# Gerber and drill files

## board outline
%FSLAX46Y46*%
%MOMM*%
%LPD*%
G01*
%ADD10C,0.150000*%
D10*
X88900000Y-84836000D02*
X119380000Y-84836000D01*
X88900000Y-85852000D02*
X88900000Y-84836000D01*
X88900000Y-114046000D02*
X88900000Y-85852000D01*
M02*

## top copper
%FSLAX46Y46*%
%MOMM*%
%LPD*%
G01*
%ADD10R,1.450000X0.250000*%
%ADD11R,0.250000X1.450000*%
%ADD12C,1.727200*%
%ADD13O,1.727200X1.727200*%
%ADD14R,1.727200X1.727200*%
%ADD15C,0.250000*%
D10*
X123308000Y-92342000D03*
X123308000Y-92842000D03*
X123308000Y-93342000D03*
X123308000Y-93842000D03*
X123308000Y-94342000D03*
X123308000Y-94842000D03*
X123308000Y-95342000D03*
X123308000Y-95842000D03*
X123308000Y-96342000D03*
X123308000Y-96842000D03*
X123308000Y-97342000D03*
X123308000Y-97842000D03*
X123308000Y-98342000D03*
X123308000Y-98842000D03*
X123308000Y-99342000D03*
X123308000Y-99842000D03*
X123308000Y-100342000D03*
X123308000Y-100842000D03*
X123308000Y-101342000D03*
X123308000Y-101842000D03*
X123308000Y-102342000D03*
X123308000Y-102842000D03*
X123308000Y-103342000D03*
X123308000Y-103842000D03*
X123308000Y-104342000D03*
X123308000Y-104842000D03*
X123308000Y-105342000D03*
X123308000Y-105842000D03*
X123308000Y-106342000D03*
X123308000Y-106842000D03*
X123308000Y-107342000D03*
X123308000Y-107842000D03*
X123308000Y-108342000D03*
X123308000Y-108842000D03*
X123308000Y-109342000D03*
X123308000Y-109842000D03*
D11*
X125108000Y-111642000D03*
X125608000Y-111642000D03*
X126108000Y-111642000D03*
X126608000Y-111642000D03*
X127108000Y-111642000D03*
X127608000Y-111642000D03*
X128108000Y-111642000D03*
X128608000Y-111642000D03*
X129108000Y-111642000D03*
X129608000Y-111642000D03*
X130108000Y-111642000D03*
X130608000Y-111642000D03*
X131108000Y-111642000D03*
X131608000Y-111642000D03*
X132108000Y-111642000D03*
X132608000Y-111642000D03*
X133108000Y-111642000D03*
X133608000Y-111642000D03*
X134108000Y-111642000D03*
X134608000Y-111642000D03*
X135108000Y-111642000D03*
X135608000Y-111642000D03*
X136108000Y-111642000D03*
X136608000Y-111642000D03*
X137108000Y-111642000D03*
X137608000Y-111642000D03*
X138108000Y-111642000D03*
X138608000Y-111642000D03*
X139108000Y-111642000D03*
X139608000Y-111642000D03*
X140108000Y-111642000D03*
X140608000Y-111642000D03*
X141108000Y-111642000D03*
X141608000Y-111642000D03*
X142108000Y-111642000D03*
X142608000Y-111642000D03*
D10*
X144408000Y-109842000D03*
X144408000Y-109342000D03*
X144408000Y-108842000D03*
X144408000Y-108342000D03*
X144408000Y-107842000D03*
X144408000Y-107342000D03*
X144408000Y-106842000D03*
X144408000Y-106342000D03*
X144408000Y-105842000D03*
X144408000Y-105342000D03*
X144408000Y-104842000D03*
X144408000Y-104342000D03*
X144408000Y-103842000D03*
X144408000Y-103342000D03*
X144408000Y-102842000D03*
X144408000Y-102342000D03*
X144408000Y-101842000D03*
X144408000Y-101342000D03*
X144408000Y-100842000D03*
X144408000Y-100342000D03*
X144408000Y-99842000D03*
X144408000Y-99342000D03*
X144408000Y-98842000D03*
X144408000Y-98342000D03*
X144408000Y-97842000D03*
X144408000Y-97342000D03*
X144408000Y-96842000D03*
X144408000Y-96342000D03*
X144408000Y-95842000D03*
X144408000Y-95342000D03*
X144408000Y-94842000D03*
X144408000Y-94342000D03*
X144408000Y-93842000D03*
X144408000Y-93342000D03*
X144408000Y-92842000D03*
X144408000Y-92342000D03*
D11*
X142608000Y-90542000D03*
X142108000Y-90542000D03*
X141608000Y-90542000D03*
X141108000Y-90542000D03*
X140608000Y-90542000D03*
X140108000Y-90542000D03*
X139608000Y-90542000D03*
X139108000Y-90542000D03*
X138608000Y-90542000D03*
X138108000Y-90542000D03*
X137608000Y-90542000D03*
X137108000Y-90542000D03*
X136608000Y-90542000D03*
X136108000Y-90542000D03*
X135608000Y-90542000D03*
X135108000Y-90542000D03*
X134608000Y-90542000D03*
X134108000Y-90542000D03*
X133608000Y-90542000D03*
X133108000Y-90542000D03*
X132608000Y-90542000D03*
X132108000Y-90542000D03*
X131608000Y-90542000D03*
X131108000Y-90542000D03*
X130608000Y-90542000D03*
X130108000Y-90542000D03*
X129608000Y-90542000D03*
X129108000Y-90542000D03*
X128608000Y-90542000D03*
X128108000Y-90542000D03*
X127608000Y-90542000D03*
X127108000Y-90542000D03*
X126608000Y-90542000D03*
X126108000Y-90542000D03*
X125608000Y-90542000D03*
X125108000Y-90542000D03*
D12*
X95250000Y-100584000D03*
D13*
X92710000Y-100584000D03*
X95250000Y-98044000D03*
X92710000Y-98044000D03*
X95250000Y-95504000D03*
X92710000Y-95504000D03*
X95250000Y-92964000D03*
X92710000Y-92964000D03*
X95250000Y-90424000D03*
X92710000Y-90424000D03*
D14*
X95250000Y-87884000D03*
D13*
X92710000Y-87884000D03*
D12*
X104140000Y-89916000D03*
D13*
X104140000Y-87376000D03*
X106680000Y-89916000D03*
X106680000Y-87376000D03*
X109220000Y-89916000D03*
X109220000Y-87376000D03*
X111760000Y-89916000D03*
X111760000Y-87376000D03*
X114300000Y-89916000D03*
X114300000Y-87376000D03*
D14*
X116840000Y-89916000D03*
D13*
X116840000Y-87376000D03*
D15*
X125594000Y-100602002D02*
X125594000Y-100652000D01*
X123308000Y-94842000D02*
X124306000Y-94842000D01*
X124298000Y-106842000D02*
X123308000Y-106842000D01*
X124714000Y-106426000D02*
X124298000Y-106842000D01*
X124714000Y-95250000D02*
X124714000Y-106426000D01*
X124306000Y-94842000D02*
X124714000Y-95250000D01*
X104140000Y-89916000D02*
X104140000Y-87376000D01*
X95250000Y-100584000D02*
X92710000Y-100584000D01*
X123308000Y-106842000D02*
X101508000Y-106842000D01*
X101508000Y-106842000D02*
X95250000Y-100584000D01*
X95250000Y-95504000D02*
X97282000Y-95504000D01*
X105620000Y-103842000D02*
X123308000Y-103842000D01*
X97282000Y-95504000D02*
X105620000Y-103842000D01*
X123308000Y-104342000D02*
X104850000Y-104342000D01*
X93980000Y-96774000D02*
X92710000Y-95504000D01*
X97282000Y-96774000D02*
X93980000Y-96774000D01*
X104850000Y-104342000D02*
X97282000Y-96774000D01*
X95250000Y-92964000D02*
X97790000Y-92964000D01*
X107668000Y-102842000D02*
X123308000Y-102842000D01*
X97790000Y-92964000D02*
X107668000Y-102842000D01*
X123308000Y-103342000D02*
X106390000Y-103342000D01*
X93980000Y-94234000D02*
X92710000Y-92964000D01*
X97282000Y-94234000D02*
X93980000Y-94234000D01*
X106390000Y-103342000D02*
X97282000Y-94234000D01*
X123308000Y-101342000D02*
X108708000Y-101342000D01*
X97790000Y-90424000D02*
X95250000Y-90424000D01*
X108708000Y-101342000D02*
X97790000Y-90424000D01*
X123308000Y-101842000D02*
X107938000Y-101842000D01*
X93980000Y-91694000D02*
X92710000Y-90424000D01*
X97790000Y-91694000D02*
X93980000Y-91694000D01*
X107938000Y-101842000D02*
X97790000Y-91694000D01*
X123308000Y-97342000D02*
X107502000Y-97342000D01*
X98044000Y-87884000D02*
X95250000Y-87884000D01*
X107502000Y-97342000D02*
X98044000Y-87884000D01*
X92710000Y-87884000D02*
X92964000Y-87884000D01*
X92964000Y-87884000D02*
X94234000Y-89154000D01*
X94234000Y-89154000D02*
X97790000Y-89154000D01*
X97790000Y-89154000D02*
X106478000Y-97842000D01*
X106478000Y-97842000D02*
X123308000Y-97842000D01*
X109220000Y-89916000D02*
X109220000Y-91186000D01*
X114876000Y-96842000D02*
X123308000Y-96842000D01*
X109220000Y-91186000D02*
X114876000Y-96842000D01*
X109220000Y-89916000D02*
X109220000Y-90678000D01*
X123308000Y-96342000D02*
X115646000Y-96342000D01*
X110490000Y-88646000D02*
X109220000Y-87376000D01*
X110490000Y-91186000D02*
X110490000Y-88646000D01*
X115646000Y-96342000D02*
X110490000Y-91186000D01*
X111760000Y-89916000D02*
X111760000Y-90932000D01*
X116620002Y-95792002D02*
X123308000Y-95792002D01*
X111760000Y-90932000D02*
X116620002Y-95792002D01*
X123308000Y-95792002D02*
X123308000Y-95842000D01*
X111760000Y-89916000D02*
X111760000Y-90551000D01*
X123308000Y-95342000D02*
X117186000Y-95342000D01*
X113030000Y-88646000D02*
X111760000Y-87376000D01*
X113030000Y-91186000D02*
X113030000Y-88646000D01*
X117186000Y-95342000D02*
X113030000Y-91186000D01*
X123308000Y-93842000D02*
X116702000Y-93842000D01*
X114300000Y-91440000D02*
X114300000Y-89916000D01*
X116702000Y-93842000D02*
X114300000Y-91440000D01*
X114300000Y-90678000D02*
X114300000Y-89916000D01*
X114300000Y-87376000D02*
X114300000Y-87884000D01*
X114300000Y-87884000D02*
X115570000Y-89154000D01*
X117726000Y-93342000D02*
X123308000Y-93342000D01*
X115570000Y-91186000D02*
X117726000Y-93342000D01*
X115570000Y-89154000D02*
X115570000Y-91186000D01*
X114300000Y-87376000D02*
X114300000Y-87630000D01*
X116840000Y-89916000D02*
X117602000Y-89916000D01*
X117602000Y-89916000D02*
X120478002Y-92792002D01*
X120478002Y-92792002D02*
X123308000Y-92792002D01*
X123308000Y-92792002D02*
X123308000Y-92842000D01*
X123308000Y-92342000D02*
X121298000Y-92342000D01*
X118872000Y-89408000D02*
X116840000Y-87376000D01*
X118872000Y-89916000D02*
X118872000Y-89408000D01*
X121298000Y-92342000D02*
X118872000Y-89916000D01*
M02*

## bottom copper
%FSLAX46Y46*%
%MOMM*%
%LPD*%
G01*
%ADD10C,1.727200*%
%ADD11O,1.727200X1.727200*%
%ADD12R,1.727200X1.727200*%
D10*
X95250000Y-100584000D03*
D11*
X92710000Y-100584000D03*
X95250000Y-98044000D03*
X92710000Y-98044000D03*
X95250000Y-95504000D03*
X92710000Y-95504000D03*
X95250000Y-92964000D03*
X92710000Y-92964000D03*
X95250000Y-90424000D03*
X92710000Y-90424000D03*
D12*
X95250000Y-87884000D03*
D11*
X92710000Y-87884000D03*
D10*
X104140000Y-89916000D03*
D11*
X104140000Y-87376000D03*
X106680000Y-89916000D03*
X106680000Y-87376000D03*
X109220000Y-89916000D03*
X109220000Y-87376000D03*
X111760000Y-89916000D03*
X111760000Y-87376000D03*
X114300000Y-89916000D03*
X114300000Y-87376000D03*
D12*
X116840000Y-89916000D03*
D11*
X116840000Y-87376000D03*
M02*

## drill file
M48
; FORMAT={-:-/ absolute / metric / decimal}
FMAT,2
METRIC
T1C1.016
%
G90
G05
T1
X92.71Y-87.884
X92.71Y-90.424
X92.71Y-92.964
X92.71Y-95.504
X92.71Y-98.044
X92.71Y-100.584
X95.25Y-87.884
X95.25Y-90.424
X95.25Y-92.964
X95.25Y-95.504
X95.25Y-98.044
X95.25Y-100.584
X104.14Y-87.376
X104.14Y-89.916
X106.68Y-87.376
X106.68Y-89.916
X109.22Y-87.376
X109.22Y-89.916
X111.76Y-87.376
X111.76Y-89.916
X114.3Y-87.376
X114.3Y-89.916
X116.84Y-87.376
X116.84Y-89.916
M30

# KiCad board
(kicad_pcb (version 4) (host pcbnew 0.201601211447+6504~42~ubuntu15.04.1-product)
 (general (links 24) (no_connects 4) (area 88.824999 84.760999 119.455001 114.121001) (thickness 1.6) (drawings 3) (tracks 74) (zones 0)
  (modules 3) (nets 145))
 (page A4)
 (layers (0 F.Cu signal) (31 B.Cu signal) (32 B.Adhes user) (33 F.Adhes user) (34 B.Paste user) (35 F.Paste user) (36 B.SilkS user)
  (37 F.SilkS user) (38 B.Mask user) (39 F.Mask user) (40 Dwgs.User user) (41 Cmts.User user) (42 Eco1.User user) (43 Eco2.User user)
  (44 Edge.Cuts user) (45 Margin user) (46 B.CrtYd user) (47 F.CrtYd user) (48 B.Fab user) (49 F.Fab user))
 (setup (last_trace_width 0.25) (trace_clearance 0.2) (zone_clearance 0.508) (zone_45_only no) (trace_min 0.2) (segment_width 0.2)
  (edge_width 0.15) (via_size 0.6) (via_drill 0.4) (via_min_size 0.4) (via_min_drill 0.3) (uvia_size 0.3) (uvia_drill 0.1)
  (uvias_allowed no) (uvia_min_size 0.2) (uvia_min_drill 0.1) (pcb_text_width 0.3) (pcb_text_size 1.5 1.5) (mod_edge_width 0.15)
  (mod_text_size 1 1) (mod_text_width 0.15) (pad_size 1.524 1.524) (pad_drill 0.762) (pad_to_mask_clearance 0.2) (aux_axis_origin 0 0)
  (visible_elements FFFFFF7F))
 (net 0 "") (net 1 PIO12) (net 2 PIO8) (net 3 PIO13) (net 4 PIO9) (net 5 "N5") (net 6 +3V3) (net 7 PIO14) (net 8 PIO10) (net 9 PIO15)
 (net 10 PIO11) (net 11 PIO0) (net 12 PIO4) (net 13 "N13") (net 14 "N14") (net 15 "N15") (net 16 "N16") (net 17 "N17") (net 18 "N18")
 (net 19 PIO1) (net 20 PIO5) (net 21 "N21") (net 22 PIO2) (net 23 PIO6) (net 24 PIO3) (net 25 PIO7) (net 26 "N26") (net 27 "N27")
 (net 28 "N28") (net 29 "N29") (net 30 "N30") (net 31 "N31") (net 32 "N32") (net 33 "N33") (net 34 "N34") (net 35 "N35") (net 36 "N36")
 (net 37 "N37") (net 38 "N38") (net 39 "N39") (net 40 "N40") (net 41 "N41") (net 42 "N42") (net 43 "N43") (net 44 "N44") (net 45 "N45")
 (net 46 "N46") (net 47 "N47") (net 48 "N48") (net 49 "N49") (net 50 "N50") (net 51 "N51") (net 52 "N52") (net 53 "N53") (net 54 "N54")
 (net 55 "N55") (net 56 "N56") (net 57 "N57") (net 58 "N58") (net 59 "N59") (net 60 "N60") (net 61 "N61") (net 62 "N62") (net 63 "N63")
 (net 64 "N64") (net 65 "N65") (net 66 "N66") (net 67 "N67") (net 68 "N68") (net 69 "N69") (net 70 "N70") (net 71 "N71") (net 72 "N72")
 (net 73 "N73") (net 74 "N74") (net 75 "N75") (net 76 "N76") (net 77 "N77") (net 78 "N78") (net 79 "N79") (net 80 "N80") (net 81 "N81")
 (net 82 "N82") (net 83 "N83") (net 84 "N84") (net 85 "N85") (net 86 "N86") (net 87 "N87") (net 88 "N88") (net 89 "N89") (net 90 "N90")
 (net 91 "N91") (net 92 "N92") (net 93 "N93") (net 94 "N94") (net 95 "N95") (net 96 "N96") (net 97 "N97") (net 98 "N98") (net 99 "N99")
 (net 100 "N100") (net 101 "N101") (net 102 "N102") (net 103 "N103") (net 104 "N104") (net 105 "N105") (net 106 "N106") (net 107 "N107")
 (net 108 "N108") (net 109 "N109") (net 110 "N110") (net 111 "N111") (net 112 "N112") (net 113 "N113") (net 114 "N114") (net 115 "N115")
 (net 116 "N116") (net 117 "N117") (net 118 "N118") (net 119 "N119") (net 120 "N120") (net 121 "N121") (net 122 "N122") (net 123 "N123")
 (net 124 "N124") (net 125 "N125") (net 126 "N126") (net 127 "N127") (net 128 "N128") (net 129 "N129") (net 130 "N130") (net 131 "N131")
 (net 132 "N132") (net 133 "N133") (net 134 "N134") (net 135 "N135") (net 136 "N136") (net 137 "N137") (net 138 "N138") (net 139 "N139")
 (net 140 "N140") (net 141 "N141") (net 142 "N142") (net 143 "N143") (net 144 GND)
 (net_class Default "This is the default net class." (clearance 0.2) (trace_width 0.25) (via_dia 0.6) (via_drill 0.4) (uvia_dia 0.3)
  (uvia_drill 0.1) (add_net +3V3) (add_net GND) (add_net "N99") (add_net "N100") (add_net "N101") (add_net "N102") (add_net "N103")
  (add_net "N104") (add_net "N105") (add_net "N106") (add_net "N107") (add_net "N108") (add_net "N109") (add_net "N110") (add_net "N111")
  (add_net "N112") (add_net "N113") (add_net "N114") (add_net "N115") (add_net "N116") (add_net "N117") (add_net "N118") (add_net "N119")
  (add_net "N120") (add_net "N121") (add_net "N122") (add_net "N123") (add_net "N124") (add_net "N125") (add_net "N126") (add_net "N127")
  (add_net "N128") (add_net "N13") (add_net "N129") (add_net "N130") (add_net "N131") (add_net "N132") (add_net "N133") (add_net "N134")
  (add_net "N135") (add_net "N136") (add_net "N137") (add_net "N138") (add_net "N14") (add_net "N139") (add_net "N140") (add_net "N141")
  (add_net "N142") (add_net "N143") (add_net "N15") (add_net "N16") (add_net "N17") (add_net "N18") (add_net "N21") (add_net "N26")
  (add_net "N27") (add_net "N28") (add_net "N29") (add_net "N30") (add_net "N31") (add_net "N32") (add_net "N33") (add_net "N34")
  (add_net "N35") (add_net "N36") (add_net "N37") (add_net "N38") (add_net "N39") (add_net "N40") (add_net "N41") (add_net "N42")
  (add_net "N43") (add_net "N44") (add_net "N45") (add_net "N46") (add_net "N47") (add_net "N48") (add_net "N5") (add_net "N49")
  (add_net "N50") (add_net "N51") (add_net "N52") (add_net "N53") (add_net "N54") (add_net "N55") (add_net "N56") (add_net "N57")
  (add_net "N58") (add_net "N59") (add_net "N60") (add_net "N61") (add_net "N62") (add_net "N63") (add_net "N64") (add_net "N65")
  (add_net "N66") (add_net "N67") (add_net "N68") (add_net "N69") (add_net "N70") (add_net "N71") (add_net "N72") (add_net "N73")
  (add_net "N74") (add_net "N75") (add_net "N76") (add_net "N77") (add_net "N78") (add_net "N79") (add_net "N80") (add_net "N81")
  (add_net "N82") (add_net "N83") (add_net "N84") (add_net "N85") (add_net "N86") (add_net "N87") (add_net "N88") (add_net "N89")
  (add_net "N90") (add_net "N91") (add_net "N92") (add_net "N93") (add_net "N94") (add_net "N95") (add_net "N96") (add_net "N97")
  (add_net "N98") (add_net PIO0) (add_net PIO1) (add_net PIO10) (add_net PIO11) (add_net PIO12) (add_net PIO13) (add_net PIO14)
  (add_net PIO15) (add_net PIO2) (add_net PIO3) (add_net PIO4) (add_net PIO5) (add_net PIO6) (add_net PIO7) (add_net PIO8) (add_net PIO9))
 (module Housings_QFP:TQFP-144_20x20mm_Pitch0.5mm (layer F.Cu) (at 133.858 101.092)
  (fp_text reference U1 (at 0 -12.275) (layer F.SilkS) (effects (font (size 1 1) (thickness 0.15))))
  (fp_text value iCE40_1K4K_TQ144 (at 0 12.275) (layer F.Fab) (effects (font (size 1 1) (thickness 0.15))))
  (pad 1 smd rect (at -10.55 -8.75) (size 1.45 0.25) (layers F.Cu F.Paste F.Mask) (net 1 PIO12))
  (pad 2 smd rect (at -10.55 -8.25) (size 1.45 0.25) (layers F.Cu F.Paste F.Mask) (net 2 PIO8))
  (pad 3 smd rect (at -10.55 -7.75) (size 1.45 0.25) (layers F.Cu F.Paste F.Mask) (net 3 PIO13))
  (pad 4 smd rect (at -10.55 -7.25) (size 1.45 0.25) (layers F.Cu F.Paste F.Mask) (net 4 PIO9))
  (pad 5 smd rect (at -10.55 -6.75) (size 1.45 0.25) (layers F.Cu F.Paste F.Mask) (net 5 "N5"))
  (pad 6 smd rect (at -10.55 -6.25) (size 1.45 0.25) (layers F.Cu F.Paste F.Mask) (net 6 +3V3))
  (pad 7 smd rect (at -10.55 -5.75) (size 1.45 0.25) (layers F.Cu F.Paste F.Mask) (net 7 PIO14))
  (pad 8 smd rect (at -10.55 -5.25) (size 1.45 0.25) (layers F.Cu F.Paste F.Mask) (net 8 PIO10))
  (pad 9 smd rect (at -10.55 -4.75) (size 1.45 0.25) (layers F.Cu F.Paste F.Mask) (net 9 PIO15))
  (pad 10 smd rect (at -10.55 -4.25) (size 1.45 0.25) (layers F.Cu F.Paste F.Mask) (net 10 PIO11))
  (pad 11 smd rect (at -10.55 -3.75) (size 1.45 0.25) (layers F.Cu F.Paste F.Mask) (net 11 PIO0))
  (pad 12 smd rect (at -10.55 -3.25) (size 1.45 0.25) (layers F.Cu F.Paste F.Mask) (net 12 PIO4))
  (pad 13 smd rect (at -10.55 -2.75) (size 1.45 0.25) (layers F.Cu F.Paste F.Mask) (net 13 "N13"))
  (pad 14 smd rect (at -10.55 -2.25) (size 1.45 0.25) (layers F.Cu F.Paste F.Mask) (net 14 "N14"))
  (pad 15 smd rect (at -10.55 -1.75) (size 1.45 0.25) (layers F.Cu F.Paste F.Mask) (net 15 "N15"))
  (pad 16 smd rect (at -10.55 -1.25) (size 1.45 0.25) (layers F.Cu F.Paste F.Mask) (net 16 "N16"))
  (pad 17 smd rect (at -10.55 -0.75) (size 1.45 0.25) (layers F.Cu F.Paste F.Mask) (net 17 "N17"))
  (pad 18 smd rect (at -10.55 -0.25) (size 1.45 0.25) (layers F.Cu F.Paste F.Mask) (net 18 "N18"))
  (pad 19 smd rect (at -10.55 0.25) (size 1.45 0.25) (layers F.Cu F.Paste F.Mask) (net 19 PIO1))
  (pad 20 smd rect (at -10.55 0.75) (size 1.45 0.25) (layers F.Cu F.Paste F.Mask) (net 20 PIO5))
  (pad 21 smd rect (at -10.55 1.25) (size 1.45 0.25) (layers F.Cu F.Paste F.Mask) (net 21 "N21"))
  (pad 22 smd rect (at -10.55 1.75) (size 1.45 0.25) (layers F.Cu F.Paste F.Mask) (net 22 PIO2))
  (pad 23 smd rect (at -10.55 2.25) (size 1.45 0.25) (layers F.Cu F.Paste F.Mask) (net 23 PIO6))
  (pad 24 smd rect (at -10.55 2.75) (size 1.45 0.25) (layers F.Cu F.Paste F.Mask) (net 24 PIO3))
  (pad 25 smd rect (at -10.55 3.25) (size 1.45 0.25) (layers F.Cu F.Paste F.Mask) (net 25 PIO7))
  (pad 26 smd rect (at -10.55 3.75) (size 1.45 0.25) (layers F.Cu F.Paste F.Mask) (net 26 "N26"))
  (pad 27 smd rect (at -10.55 4.25) (size 1.45 0.25) (layers F.Cu F.Paste F.Mask) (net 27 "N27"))
  (pad 28 smd rect (at -10.55 4.75) (size 1.45 0.25) (layers F.Cu F.Paste F.Mask) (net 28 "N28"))
  (pad 29 smd rect (at -10.55 5.25) (size 1.45 0.25) (layers F.Cu F.Paste F.Mask) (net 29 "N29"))
  (pad 30 smd rect (at -10.55 5.75) (size 1.45 0.25) (layers F.Cu F.Paste F.Mask) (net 6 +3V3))
  (pad 31 smd rect (at -10.55 6.25) (size 1.45 0.25) (layers F.Cu F.Paste F.Mask) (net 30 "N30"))
  (pad 32 smd rect (at -10.55 6.75) (size 1.45 0.25) (layers F.Cu F.Paste F.Mask) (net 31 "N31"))
  (pad 33 smd rect (at -10.55 7.25) (size 1.45 0.25) (layers F.Cu F.Paste F.Mask) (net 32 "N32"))
  (pad 34 smd rect (at -10.55 7.75) (size 1.45 0.25) (layers F.Cu F.Paste F.Mask) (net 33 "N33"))
  (pad 35 smd rect (at -10.55 8.25) (size 1.45 0.25) (layers F.Cu F.Paste F.Mask) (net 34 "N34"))
  (pad 36 smd rect (at -10.55 8.75) (size 1.45 0.25) (layers F.Cu F.Paste F.Mask) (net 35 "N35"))
  (pad 37 smd rect (at -8.75 10.55 90) (size 1.45 0.25) (layers F.Cu F.Paste F.Mask) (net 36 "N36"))
  (pad 38 smd rect (at -8.25 10.55 90) (size 1.45 0.25) (layers F.Cu F.Paste F.Mask) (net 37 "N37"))
  (pad 39 smd rect (at -7.75 10.55 90) (size 1.45 0.25) (layers F.Cu F.Paste F.Mask) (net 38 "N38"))
  (pad 40 smd rect (at -7.25 10.55 90) (size 1.45 0.25) (layers F.Cu F.Paste F.Mask) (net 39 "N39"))
  (pad 41 smd rect (at -6.75 10.55 90) (size 1.45 0.25) (layers F.Cu F.Paste F.Mask) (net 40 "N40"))
  (pad 42 smd rect (at -6.25 10.55 90) (size 1.45 0.25) (layers F.Cu F.Paste F.Mask) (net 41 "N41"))
  (pad 43 smd rect (at -5.75 10.55 90) (size 1.45 0.25) (layers F.Cu F.Paste F.Mask) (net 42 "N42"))
  (pad 44 smd rect (at -5.25 10.55 90) (size 1.45 0.25) (layers F.Cu F.Paste F.Mask) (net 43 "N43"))
  (pad 45 smd rect (at -4.75 10.55 90) (size 1.45 0.25) (layers F.Cu F.Paste F.Mask) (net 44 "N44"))
  (pad 46 smd rect (at -4.25 10.55 90) (size 1.45 0.25) (layers F.Cu F.Paste F.Mask) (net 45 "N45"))
  (pad 47 smd rect (at -3.75 10.55 90) (size 1.45 0.25) (layers F.Cu F.Paste F.Mask) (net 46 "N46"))
  (pad 48 smd rect (at -3.25 10.55 90) (size 1.45 0.25) (layers F.Cu F.Paste F.Mask) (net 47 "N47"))
  (pad 49 smd rect (at -2.75 10.55 90) (size 1.45 0.25) (layers F.Cu F.Paste F.Mask) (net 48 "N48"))
  (pad 50 smd rect (at -2.25 10.55 90) (size 1.45 0.25) (layers F.Cu F.Paste F.Mask) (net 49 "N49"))
  (pad 51 smd rect (at -1.75 10.55 90) (size 1.45 0.25) (layers F.Cu F.Paste F.Mask) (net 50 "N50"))
  (pad 52 smd rect (at -1.25 10.55 90) (size 1.45 0.25) (layers F.Cu F.Paste F.Mask) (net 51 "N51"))
  (pad 53 smd rect (at -0.75 10.55 90) (size 1.45 0.25) (layers F.Cu F.Paste F.Mask) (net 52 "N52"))
  (pad 54 smd rect (at -0.25 10.55 90) (size 1.45 0.25) (layers F.Cu F.Paste F.Mask) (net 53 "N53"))
  (pad 55 smd rect (at 0.25 10.55 90) (size 1.45 0.25) (layers F.Cu F.Paste F.Mask) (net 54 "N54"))
  (pad 56 smd rect (at 0.75 10.55 90) (size 1.45 0.25) (layers F.Cu F.Paste F.Mask) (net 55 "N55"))
  (pad 57 smd rect (at 1.25 10.55 90) (size 1.45 0.25) (layers F.Cu F.Paste F.Mask) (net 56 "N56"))
  (pad 58 smd rect (at 1.75 10.55 90) (size 1.45 0.25) (layers F.Cu F.Paste F.Mask) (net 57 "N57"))
  (pad 59 smd rect (at 2.25 10.55 90) (size 1.45 0.25) (layers F.Cu F.Paste F.Mask) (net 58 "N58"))
  (pad 60 smd rect (at 2.75 10.55 90) (size 1.45 0.25) (layers F.Cu F.Paste F.Mask) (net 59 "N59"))
  (pad 61 smd rect (at 3.25 10.55 90) (size 1.45 0.25) (layers F.Cu F.Paste F.Mask) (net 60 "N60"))
  (pad 62 smd rect (at 3.75 10.55 90) (size 1.45 0.25) (layers F.Cu F.Paste F.Mask) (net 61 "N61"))
  (pad 63 smd rect (at 4.25 10.55 90) (size 1.45 0.25) (layers F.Cu F.Paste F.Mask) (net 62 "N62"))
  (pad 64 smd rect (at 4.75 10.55 90) (size 1.45 0.25) (layers F.Cu F.Paste F.Mask) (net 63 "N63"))
  (pad 65 smd rect (at 5.25 10.55 90) (size 1.45 0.25) (layers F.Cu F.Paste F.Mask) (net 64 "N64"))
  (pad 66 smd rect (at 5.75 10.55 90) (size 1.45 0.25) (layers F.Cu F.Paste F.Mask) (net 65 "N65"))
  (pad 67 smd rect (at 6.25 10.55 90) (size 1.45 0.25) (layers F.Cu F.Paste F.Mask) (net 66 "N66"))
  (pad 68 smd rect (at 6.75 10.55 90) (size 1.45 0.25) (layers F.Cu F.Paste F.Mask) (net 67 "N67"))
  (pad 69 smd rect (at 7.25 10.55 90) (size 1.45 0.25) (layers F.Cu F.Paste F.Mask) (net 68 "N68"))
  (pad 70 smd rect (at 7.75 10.55 90) (size 1.45 0.25) (layers F.Cu F.Paste F.Mask) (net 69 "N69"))
  (pad 71 smd rect (at 8.25 10.55 90) (size 1.45 0.25) (layers F.Cu F.Paste F.Mask) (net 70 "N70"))
  (pad 72 smd rect (at 8.75 10.55 90) (size 1.45 0.25) (layers F.Cu F.Paste F.Mask) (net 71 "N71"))
  (pad 73 smd rect (at 10.55 8.75) (size 1.45 0.25) (layers F.Cu F.Paste F.Mask) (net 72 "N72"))
  (pad 74 smd rect (at 10.55 8.25) (size 1.45 0.25) (layers F.Cu F.Paste F.Mask) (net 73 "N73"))
  (pad 75 smd rect (at 10.55 7.75) (size 1.45 0.25) (layers F.Cu F.Paste F.Mask) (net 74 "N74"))
  (pad 76 smd rect (at 10.55 7.25) (size 1.45 0.25) (layers F.Cu F.Paste F.Mask) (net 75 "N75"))
  (pad 77 smd rect (at 10.55 6.75) (size 1.45 0.25) (layers F.Cu F.Paste F.Mask) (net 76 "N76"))
  (pad 78 smd rect (at 10.55 6.25) (size 1.45 0.25) (layers F.Cu F.Paste F.Mask) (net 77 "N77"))
  (pad 79 smd rect (at 10.55 5.75) (size 1.45 0.25) (layers F.Cu F.Paste F.Mask) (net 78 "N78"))
  (pad 80 smd rect (at 10.55 5.25) (size 1.45 0.25) (layers F.Cu F.Paste F.Mask) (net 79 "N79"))
  (pad 81 smd rect (at 10.55 4.75) (size 1.45 0.25) (layers F.Cu F.Paste F.Mask) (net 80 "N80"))
  (pad 82 smd rect (at 10.55 4.25) (size 1.45 0.25) (layers F.Cu F.Paste F.Mask) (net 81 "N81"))
  (pad 83 smd rect (at 10.55 3.75) (size 1.45 0.25) (layers F.Cu F.Paste F.Mask) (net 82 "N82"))
  (pad 84 smd rect (at 10.55 3.25) (size 1.45 0.25) (layers F.Cu F.Paste F.Mask) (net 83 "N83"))
  (pad 85 smd rect (at 10.55 2.75) (size 1.45 0.25) (layers F.Cu F.Paste F.Mask) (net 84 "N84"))
  (pad 86 smd rect (at 10.55 2.25) (size 1.45 0.25) (layers F.Cu F.Paste F.Mask) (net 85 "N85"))
  (pad 87 smd rect (at 10.55 1.75) (size 1.45 0.25) (layers F.Cu F.Paste F.Mask) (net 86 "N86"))
  (pad 88 smd rect (at 10.55 1.25) (size 1.45 0.25) (layers F.Cu F.Paste F.Mask) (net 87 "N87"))
  (pad 89 smd rect (at 10.55 0.75) (size 1.45 0.25) (layers F.Cu F.Paste F.Mask) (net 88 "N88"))
  (pad 90 smd rect (at 10.55 0.25) (size 1.45 0.25) (layers F.Cu F.Paste F.Mask) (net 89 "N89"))
  (pad 91 smd rect (at 10.55 -0.25) (size 1.45 0.25) (layers F.Cu F.Paste F.Mask) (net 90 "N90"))
  (pad 92 smd rect (at 10.55 -0.75) (size 1.45 0.25) (layers F.Cu F.Paste F.Mask) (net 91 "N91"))
  (pad 93 smd rect (at 10.55 -1.25) (size 1.45 0.25) (layers F.Cu F.Paste F.Mask) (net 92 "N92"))
  (pad 94 smd rect (at 10.55 -1.75) (size 1.45 0.25) (layers F.Cu F.Paste F.Mask) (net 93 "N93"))
  (pad 95 smd rect (at 10.55 -2.25) (size 1.45 0.25) (layers F.Cu F.Paste F.Mask) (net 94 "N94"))
  (pad 96 smd rect (at 10.55 -2.75) (size 1.45 0.25) (layers F.Cu F.Paste F.Mask) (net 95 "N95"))
  (pad 97 smd rect (at 10.55 -3.25) (size 1.45 0.25) (layers F.Cu F.Paste F.Mask) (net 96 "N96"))
  (pad 98 smd rect (at 10.55 -3.75) (size 1.45 0.25) (layers F.Cu F.Paste F.Mask) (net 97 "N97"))
  (pad 99 smd rect (at 10.55 -4.25) (size 1.45 0.25) (layers F.Cu F.Paste F.Mask) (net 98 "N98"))
  (pad 100 smd rect (at 10.55 -4.75) (size 1.45 0.25) (layers F.Cu F.Paste F.Mask) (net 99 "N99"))
  (pad 101 smd rect (at 10.55 -5.25) (size 1.45 0.25) (layers F.Cu F.Paste F.Mask) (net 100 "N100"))
  (pad 102 smd rect (at 10.55 -5.75) (size 1.45 0.25) (layers F.Cu F.Paste F.Mask) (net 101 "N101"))
  (pad 103 smd rect (at 10.55 -6.25) (size 1.45 0.25) (layers F.Cu F.Paste F.Mask) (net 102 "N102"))
  (pad 104 smd rect (at 10.55 -6.75) (size 1.45 0.25) (layers F.Cu F.Paste F.Mask) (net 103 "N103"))
  (pad 105 smd rect (at 10.55 -7.25) (size 1.45 0.25) (layers F.Cu F.Paste F.Mask) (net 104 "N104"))
  (pad 106 smd rect (at 10.55 -7.75) (size 1.45 0.25) (layers F.Cu F.Paste F.Mask) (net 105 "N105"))
  (pad 107 smd rect (at 10.55 -8.25) (size 1.45 0.25) (layers F.Cu F.Paste F.Mask) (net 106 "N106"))
  (pad 108 smd rect (at 10.55 -8.75) (size 1.45 0.25) (layers F.Cu F.Paste F.Mask) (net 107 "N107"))
  (pad 109 smd rect (at 8.75 -10.55 90) (size 1.45 0.25) (layers F.Cu F.Paste F.Mask) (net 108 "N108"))
  (pad 110 smd rect (at 8.25 -10.55 90) (size 1.45 0.25) (layers F.Cu F.Paste F.Mask) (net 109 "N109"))
  (pad 111 smd rect (at 7.75 -10.55 90) (size 1.45 0.25) (layers F.Cu F.Paste F.Mask) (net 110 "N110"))
  (pad 112 smd rect (at 7.25 -10.55 90) (size 1.45 0.25) (layers F.Cu F.Paste F.Mask) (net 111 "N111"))
  (pad 113 smd rect (at 6.75 -10.55 90) (size 1.45 0.25) (layers F.Cu F.Paste F.Mask) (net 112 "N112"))
  (pad 114 smd rect (at 6.25 -10.55 90) (size 1.45 0.25) (layers F.Cu F.Paste F.Mask) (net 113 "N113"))
  (pad 115 smd rect (at 5.75 -10.55 90) (size 1.45 0.25) (layers F.Cu F.Paste F.Mask) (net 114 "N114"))
  (pad 116 smd rect (at 5.25 -10.55 90) (size 1.45 0.25) (layers F.Cu F.Paste F.Mask) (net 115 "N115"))
  (pad 117 smd rect (at 4.75 -10.55 90) (size 1.45 0.25) (layers F.Cu F.Paste F.Mask) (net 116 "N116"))
  (pad 118 smd rect (at 4.25 -10.55 90) (size 1.45 0.25) (layers F.Cu F.Paste F.Mask) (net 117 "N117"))
  (pad 119 smd rect (at 3.75 -10.55 90) (size 1.45 0.25) (layers F.Cu F.Paste F.Mask) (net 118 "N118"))
  (pad 120 smd rect (at 3.25 -10.55 90) (size 1.45 0.25) (layers F.Cu F.Paste F.Mask) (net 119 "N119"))
  (pad 121 smd rect (at 2.75 -10.55 90) (size 1.45 0.25) (layers F.Cu F.Paste F.Mask) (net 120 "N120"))
  (pad 122 smd rect (at 2.25 -10.55 90) (size 1.45 0.25) (layers F.Cu F.Paste F.Mask) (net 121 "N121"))
  (pad 123 smd rect (at 1.75 -10.55 90) (size 1.45 0.25) (layers F.Cu F.Paste F.Mask) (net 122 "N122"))
  (pad 124 smd rect (at 1.25 -10.55 90) (size 1.45 0.25) (layers F.Cu F.Paste F.Mask) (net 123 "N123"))
  (pad 125 smd rect (at 0.75 -10.55 90) (size 1.45 0.25) (layers F.Cu F.Paste F.Mask) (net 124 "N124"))
  (pad 126 smd rect (at 0.25 -10.55 90) (size 1.45 0.25) (layers F.Cu F.Paste F.Mask) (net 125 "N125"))
  (pad 127 smd rect (at -0.25 -10.55 90) (size 1.45 0.25) (layers F.Cu F.Paste F.Mask) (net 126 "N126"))
  (pad 128 smd rect (at -0.75 -10.55 90) (size 1.45 0.25) (layers F.Cu F.Paste F.Mask) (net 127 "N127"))
  (pad 129 smd rect (at -1.25 -10.55 90) (size 1.45 0.25) (layers F.Cu F.Paste F.Mask) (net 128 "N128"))
  (pad 130 smd rect (at -1.75 -10.55 90) (size 1.45 0.25) (layers F.Cu F.Paste F.Mask) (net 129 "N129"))
  (pad 131 smd rect (at -2.25 -10.55 90) (size 1.45 0.25) (layers F.Cu F.Paste F.Mask) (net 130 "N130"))
  (pad 132 smd rect (at -2.75 -10.55 90) (size 1.45 0.25) (layers F.Cu F.Paste F.Mask) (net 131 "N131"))
  (pad 133 smd rect (at -3.25 -10.55 90) (size 1.45 0.25) (layers F.Cu F.Paste F.Mask) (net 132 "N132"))
  (pad 134 smd rect (at -3.75 -10.55 90) (size 1.45 0.25) (layers F.Cu F.Paste F.Mask) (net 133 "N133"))
  (pad 135 smd rect (at -4.25 -10.55 90) (size 1.45 0.25) (layers F.Cu F.Paste F.Mask) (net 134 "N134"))
  (pad 136 smd rect (at -4.75 -10.55 90) (size 1.45 0.25) (layers F.Cu F.Paste F.Mask) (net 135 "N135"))
  (pad 137 smd rect (at -5.25 -10.55 90) (size 1.45 0.25) (layers F.Cu F.Paste F.Mask) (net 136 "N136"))
  (pad 138 smd rect (at -5.75 -10.55 90) (size 1.45 0.25) (layers F.Cu F.Paste F.Mask) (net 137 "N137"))
  (pad 139 smd rect (at -6.25 -10.55 90) (size 1.45 0.25) (layers F.Cu F.Paste F.Mask) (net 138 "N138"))
  (pad 140 smd rect (at -6.75 -10.55 90) (size 1.45 0.25) (layers F.Cu F.Paste F.Mask) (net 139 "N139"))
  (pad 141 smd rect (at -7.25 -10.55 90) (size 1.45 0.25) (layers F.Cu F.Paste F.Mask) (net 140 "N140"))
  (pad 142 smd rect (at -7.75 -10.55 90) (size 1.45 0.25) (layers F.Cu F.Paste F.Mask) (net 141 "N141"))
  (pad 143 smd rect (at -8.25 -10.55 90) (size 1.45 0.25) (layers F.Cu F.Paste F.Mask) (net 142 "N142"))
  (pad 144 smd rect (at -8.75 -10.55 90) (size 1.45 0.25) (layers F.Cu F.Paste F.Mask) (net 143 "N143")))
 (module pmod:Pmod (layer F.Cu) (at 88.9 86.614)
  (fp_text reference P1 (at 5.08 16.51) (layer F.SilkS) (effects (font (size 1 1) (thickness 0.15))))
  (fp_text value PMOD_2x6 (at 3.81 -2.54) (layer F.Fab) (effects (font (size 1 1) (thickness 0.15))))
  (pad 6 thru_hole circle (at 6.35 13.97 180) (size 1.7272 1.7272) (drill 1.016) (layers *.Cu *.Mask F.SilkS) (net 6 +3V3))
  (pad 12 thru_hole oval (at 3.81 13.97 180) (size 1.7272 1.7272) (drill 1.016) (layers *.Cu *.Mask F.SilkS) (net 6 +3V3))
  (pad 5 thru_hole oval (at 6.35 11.43 180) (size 1.7272 1.7272) (drill 1.016) (layers *.Cu *.Mask F.SilkS) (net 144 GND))
  (pad 11 thru_hole oval (at 3.81 11.43 180) (size 1.7272 1.7272) (drill 1.016) (layers *.Cu *.Mask F.SilkS) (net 144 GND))
  (pad 4 thru_hole oval (at 6.35 8.89 180) (size 1.7272 1.7272) (drill 1.016) (layers *.Cu *.Mask F.SilkS) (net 24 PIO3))
  (pad 10 thru_hole oval (at 3.81 8.89 180) (size 1.7272 1.7272) (drill 1.016) (layers *.Cu *.Mask F.SilkS) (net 25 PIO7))
  (pad 3 thru_hole oval (at 6.35 6.35 180) (size 1.7272 1.7272) (drill 1.016) (layers *.Cu *.Mask F.SilkS) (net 22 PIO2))
  (pad 9 thru_hole oval (at 3.81 6.35 180) (size 1.7272 1.7272) (drill 1.016) (layers *.Cu *.Mask F.SilkS) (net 23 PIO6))
  (pad 2 thru_hole oval (at 6.35 3.81 180) (size 1.7272 1.7272) (drill 1.016) (layers *.Cu *.Mask F.SilkS) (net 19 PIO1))
  (pad 8 thru_hole oval (at 3.81 3.81 180) (size 1.7272 1.7272) (drill 1.016) (layers *.Cu *.Mask F.SilkS) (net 20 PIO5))
  (pad 1 thru_hole rect (at 6.35 1.27 180) (size 1.7272 1.7272) (drill 1.016) (layers *.Cu *.Mask F.SilkS) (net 11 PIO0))
  (pad 7 thru_hole oval (at 3.81 1.27 180) (size 1.7272 1.7272) (drill 1.016) (layers *.Cu *.Mask F.SilkS) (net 12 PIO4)))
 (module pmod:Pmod (layer F.Cu) (at 118.11 83.566 270)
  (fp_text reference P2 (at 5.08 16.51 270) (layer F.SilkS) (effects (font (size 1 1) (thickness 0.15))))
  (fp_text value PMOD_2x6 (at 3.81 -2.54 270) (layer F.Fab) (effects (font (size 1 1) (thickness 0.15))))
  (pad 6 thru_hole circle (at 6.35 13.97 90) (size 1.7272 1.7272) (drill 1.016) (layers *.Cu *.Mask F.SilkS) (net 6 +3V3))
  (pad 12 thru_hole oval (at 3.81 13.97 90) (size 1.7272 1.7272) (drill 1.016) (layers *.Cu *.Mask F.SilkS) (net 6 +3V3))
  (pad 5 thru_hole oval (at 6.35 11.43 90) (size 1.7272 1.7272) (drill 1.016) (layers *.Cu *.Mask F.SilkS) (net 144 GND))
  (pad 11 thru_hole oval (at 3.81 11.43 90) (size 1.7272 1.7272) (drill 1.016) (layers *.Cu *.Mask F.SilkS) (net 144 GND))
  (pad 4 thru_hole oval (at 6.35 8.89 90) (size 1.7272 1.7272) (drill 1.016) (layers *.Cu *.Mask F.SilkS) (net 10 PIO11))
  (pad 10 thru_hole oval (at 3.81 8.89 90) (size 1.7272 1.7272) (drill 1.016) (layers *.Cu *.Mask F.SilkS) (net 9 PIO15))
  (pad 3 thru_hole oval (at 6.35 6.35 90) (size 1.7272 1.7272) (drill 1.016) (layers *.Cu *.Mask F.SilkS) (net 8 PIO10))
  (pad 9 thru_hole oval (at 3.81 6.35 90) (size 1.7272 1.7272) (drill 1.016) (layers *.Cu *.Mask F.SilkS) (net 7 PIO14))
  (pad 2 thru_hole oval (at 6.35 3.81 90) (size 1.7272 1.7272) (drill 1.016) (layers *.Cu *.Mask F.SilkS) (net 4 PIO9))
  (pad 8 thru_hole oval (at 3.81 3.81 90) (size 1.7272 1.7272) (drill 1.016) (layers *.Cu *.Mask F.SilkS) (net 3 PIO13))
  (pad 1 thru_hole rect (at 6.35 1.27 90) (size 1.7272 1.7272) (drill 1.016) (layers *.Cu *.Mask F.SilkS) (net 2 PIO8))
  (pad 7 thru_hole oval (at 3.81 1.27 90) (size 1.7272 1.7272) (drill 1.016) (layers *.Cu *.Mask F.SilkS) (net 1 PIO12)))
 (gr_line (start 88.9 84.836) (end 119.38 84.836) (angle 90) (layer Edge.Cuts) (width 0.15))
 (gr_line (start 88.9 85.852) (end 88.9 84.836) (angle 90) (layer Edge.Cuts) (width 0.15))
 (gr_line (start 88.9 114.046) (end 88.9 85.852) (angle 90) (layer Edge.Cuts) (width 0.15))
 (segment (start 125.594 100.602002) (end 125.594 100.652) (width 0.25) (layer F.Cu) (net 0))
 (segment (start 123.308 94.842) (end 124.306 94.842) (width 0.25) (layer F.Cu) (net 6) (status 400000))
 (segment (start 124.298 106.842) (end 123.308 106.842) (width 0.25) (layer F.Cu) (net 6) (status 800000))
 (segment (start 124.714 106.426) (end 124.298 106.842) (width 0.25) (layer F.Cu) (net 6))
 (segment (start 124.714 95.25) (end 124.714 106.426) (width 0.25) (layer F.Cu) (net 6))
 (segment (start 124.306 94.842) (end 124.714 95.25) (width 0.25) (layer F.Cu) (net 6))
 (segment (start 104.14 89.916) (end 104.14 87.376) (width 0.25) (layer F.Cu) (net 6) (status C00000))
 (segment (start 95.25 100.584) (end 92.71 100.584) (width 0.25) (layer F.Cu) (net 6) (status C00000))
 (segment (start 123.308 106.842) (end 101.508 106.842) (width 0.25) (layer F.Cu) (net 6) (status 400000))
 (segment (start 101.508 106.842) (end 95.25 100.584) (width 0.25) (layer F.Cu) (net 6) (status 800000))
 (segment (start 95.25 95.504) (end 97.282 95.504) (width 0.25) (layer F.Cu) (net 24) (status 400000))
 (segment (start 105.62 103.842) (end 123.308 103.842) (width 0.25) (layer F.Cu) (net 24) (status 800000))
 (segment (start 97.282 95.504) (end 105.62 103.842) (width 0.25) (layer F.Cu) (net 24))
 (segment (start 123.308 104.342) (end 104.85 104.342) (width 0.25) (layer F.Cu) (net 25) (status 400000))
 (segment (start 93.98 96.774) (end 92.71 95.504) (width 0.25) (layer F.Cu) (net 25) (status 800000))
 (segment (start 97.282 96.774) (end 93.98 96.774) (width 0.25) (layer F.Cu) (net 25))
 (segment (start 104.85 104.342) (end 97.282 96.774) (width 0.25) (layer F.Cu) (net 25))
 (segment (start 95.25 92.964) (end 97.79 92.964) (width 0.25) (layer F.Cu) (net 22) (status 400000))
 (segment (start 107.668 102.842) (end 123.308 102.842) (width 0.25) (layer F.Cu) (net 22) (status 800000))
 (segment (start 97.79 92.964) (end 107.668 102.842) (width 0.25) (layer F.Cu) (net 22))
 (segment (start 123.308 103.342) (end 106.39 103.342) (width 0.25) (layer F.Cu) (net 23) (status 400000))
 (segment (start 93.98 94.234) (end 92.71 92.964) (width 0.25) (layer F.Cu) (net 23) (status 800000))
 (segment (start 97.282 94.234) (end 93.98 94.234) (width 0.25) (layer F.Cu) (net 23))
 (segment (start 106.39 103.342) (end 97.282 94.234) (width 0.25) (layer F.Cu) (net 23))
 (segment (start 123.308 101.342) (end 108.708 101.342) (width 0.25) (layer F.Cu) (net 19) (status 400000))
 (segment (start 97.79 90.424) (end 95.25 90.424) (width 0.25) (layer F.Cu) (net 19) (status 800000))
 (segment (start 108.708 101.342) (end 97.79 90.424) (width 0.25) (layer F.Cu) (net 19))
 (segment (start 123.308 101.842) (end 107.938 101.842) (width 0.25) (layer F.Cu) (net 20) (status 400000))
 (segment (start 93.98 91.694) (end 92.71 90.424) (width 0.25) (layer F.Cu) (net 20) (status 800000))
 (segment (start 97.79 91.694) (end 93.98 91.694) (width 0.25) (layer F.Cu) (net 20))
 (segment (start 107.938 101.842) (end 97.79 91.694) (width 0.25) (layer F.Cu) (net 20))
 (segment (start 123.308 97.342) (end 107.502 97.342) (width 0.25) (layer F.Cu) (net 11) (status 400000))
 (segment (start 98.044 87.884) (end 95.25 87.884) (width 0.25) (layer F.Cu) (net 11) (status 800000))
 (segment (start 107.502 97.342) (end 98.044 87.884) (width 0.25) (layer F.Cu) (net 11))
 (segment (start 92.71 87.884) (end 92.964 87.884) (width 0.25) (layer F.Cu) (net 12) (status C00000))
 (segment (start 92.964 87.884) (end 94.234 89.154) (width 0.25) (layer F.Cu) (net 12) (status 400000))
 (segment (start 94.234 89.154) (end 97.79 89.154) (width 0.25) (layer F.Cu) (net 12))
 (segment (start 97.79 89.154) (end 106.478 97.842) (width 0.25) (layer F.Cu) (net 12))
 (segment (start 106.478 97.842) (end 123.308 97.842) (width 0.25) (layer F.Cu) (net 12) (status 800000))
 (segment (start 109.22 89.916) (end 109.22 91.186) (width 0.25) (layer F.Cu) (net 10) (status 400000))
 (segment (start 114.876 96.842) (end 123.308 96.842) (width 0.25) (layer F.Cu) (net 10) (status 800000))
 (segment (start 109.22 91.186) (end 114.876 96.842) (width 0.25) (layer F.Cu) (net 10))
 (segment (start 109.22 89.916) (end 109.22 90.678) (width 0.25) (layer F.Cu) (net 10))
 (segment (start 123.308 96.342) (end 115.646 96.342) (width 0.25) (layer F.Cu) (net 9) (status 400000))
 (segment (start 110.49 88.646) (end 109.22 87.376) (width 0.25) (layer F.Cu) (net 9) (status 800000))
 (segment (start 110.49 91.186) (end 110.49 88.646) (width 0.25) (layer F.Cu) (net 9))
 (segment (start 115.646 96.342) (end 110.49 91.186) (width 0.25) (layer F.Cu) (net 9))
 (segment (start 111.76 89.916) (end 111.76 90.932) (width 0.25) (layer F.Cu) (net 8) (status 400000))
 (segment (start 116.620002 95.792002) (end 123.308 95.792002) (width 0.25) (layer F.Cu) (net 8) (status 800000))
 (segment (start 111.76 90.932) (end 116.620002 95.792002) (width 0.25) (layer F.Cu) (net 8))
 (segment (start 123.308 95.792002) (end 123.308 95.842) (width 0.25) (layer F.Cu) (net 8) (status C00000))
 (segment (start 111.76 89.916) (end 111.76 90.551) (width 0.25) (layer F.Cu) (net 8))
 (segment (start 123.308 95.342) (end 117.186 95.342) (width 0.25) (layer F.Cu) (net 7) (status 400000))
 (segment (start 113.03 88.646) (end 111.76 87.376) (width 0.25) (layer F.Cu) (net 7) (status 800000))
 (segment (start 113.03 91.186) (end 113.03 88.646) (width 0.25) (layer F.Cu) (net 7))
 (segment (start 117.186 95.342) (end 113.03 91.186) (width 0.25) (layer F.Cu) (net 7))
 (segment (start 123.308 93.842) (end 116.702 93.842) (width 0.25) (layer F.Cu) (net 4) (status 400000))
 (segment (start 114.3 91.44) (end 114.3 89.916) (width 0.25) (layer F.Cu) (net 4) (status 800000))
 (segment (start 116.702 93.842) (end 114.3 91.44) (width 0.25) (layer F.Cu) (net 4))
 (segment (start 114.3 90.678) (end 114.3 89.916) (width 0.25) (layer F.Cu) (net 4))
 (segment (start 114.3 87.376) (end 114.3 87.884) (width 0.25) (layer F.Cu) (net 3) (status C00000))
 (segment (start 114.3 87.884) (end 115.57 89.154) (width 0.25) (layer F.Cu) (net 3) (status 400000))
 (segment (start 117.726 93.342) (end 123.308 93.342) (width 0.25) (layer F.Cu) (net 3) (status 800000))
 (segment (start 115.57 91.186) (end 117.726 93.342) (width 0.25) (layer F.Cu) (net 3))
 (segment (start 115.57 89.154) (end 115.57 91.186) (width 0.25) (layer F.Cu) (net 3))
 (segment (start 114.3 87.376) (end 114.3 87.63) (width 0.25) (layer F.Cu) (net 3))
 (segment (start 116.84 89.916) (end 117.602 89.916) (width 0.25) (layer F.Cu) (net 2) (status C00000))
 (segment (start 117.602 89.916) (end 120.478002 92.792002) (width 0.25) (layer F.Cu) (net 2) (status 400000))
 (segment (start 120.478002 92.792002) (end 123.308 92.792002) (width 0.25) (layer F.Cu) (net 2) (status 800000))
 (segment (start 123.308 92.792002) (end 123.308 92.842) (width 0.25) (layer F.Cu) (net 2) (status C00000))
 (segment (start 123.308 92.342) (end 121.298 92.342) (width 0.25) (layer F.Cu) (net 1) (status 400000))
 (segment (start 118.872 89.408) (end 116.84 87.376) (width 0.25) (layer F.Cu) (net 1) (status 800000))
 (segment (start 118.872 89.916) (end 118.872 89.408) (width 0.25) (layer F.Cu) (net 1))
 (segment (start 121.298 92.342) (end 118.872 89.916) (width 0.25) (layer F.Cu) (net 1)))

